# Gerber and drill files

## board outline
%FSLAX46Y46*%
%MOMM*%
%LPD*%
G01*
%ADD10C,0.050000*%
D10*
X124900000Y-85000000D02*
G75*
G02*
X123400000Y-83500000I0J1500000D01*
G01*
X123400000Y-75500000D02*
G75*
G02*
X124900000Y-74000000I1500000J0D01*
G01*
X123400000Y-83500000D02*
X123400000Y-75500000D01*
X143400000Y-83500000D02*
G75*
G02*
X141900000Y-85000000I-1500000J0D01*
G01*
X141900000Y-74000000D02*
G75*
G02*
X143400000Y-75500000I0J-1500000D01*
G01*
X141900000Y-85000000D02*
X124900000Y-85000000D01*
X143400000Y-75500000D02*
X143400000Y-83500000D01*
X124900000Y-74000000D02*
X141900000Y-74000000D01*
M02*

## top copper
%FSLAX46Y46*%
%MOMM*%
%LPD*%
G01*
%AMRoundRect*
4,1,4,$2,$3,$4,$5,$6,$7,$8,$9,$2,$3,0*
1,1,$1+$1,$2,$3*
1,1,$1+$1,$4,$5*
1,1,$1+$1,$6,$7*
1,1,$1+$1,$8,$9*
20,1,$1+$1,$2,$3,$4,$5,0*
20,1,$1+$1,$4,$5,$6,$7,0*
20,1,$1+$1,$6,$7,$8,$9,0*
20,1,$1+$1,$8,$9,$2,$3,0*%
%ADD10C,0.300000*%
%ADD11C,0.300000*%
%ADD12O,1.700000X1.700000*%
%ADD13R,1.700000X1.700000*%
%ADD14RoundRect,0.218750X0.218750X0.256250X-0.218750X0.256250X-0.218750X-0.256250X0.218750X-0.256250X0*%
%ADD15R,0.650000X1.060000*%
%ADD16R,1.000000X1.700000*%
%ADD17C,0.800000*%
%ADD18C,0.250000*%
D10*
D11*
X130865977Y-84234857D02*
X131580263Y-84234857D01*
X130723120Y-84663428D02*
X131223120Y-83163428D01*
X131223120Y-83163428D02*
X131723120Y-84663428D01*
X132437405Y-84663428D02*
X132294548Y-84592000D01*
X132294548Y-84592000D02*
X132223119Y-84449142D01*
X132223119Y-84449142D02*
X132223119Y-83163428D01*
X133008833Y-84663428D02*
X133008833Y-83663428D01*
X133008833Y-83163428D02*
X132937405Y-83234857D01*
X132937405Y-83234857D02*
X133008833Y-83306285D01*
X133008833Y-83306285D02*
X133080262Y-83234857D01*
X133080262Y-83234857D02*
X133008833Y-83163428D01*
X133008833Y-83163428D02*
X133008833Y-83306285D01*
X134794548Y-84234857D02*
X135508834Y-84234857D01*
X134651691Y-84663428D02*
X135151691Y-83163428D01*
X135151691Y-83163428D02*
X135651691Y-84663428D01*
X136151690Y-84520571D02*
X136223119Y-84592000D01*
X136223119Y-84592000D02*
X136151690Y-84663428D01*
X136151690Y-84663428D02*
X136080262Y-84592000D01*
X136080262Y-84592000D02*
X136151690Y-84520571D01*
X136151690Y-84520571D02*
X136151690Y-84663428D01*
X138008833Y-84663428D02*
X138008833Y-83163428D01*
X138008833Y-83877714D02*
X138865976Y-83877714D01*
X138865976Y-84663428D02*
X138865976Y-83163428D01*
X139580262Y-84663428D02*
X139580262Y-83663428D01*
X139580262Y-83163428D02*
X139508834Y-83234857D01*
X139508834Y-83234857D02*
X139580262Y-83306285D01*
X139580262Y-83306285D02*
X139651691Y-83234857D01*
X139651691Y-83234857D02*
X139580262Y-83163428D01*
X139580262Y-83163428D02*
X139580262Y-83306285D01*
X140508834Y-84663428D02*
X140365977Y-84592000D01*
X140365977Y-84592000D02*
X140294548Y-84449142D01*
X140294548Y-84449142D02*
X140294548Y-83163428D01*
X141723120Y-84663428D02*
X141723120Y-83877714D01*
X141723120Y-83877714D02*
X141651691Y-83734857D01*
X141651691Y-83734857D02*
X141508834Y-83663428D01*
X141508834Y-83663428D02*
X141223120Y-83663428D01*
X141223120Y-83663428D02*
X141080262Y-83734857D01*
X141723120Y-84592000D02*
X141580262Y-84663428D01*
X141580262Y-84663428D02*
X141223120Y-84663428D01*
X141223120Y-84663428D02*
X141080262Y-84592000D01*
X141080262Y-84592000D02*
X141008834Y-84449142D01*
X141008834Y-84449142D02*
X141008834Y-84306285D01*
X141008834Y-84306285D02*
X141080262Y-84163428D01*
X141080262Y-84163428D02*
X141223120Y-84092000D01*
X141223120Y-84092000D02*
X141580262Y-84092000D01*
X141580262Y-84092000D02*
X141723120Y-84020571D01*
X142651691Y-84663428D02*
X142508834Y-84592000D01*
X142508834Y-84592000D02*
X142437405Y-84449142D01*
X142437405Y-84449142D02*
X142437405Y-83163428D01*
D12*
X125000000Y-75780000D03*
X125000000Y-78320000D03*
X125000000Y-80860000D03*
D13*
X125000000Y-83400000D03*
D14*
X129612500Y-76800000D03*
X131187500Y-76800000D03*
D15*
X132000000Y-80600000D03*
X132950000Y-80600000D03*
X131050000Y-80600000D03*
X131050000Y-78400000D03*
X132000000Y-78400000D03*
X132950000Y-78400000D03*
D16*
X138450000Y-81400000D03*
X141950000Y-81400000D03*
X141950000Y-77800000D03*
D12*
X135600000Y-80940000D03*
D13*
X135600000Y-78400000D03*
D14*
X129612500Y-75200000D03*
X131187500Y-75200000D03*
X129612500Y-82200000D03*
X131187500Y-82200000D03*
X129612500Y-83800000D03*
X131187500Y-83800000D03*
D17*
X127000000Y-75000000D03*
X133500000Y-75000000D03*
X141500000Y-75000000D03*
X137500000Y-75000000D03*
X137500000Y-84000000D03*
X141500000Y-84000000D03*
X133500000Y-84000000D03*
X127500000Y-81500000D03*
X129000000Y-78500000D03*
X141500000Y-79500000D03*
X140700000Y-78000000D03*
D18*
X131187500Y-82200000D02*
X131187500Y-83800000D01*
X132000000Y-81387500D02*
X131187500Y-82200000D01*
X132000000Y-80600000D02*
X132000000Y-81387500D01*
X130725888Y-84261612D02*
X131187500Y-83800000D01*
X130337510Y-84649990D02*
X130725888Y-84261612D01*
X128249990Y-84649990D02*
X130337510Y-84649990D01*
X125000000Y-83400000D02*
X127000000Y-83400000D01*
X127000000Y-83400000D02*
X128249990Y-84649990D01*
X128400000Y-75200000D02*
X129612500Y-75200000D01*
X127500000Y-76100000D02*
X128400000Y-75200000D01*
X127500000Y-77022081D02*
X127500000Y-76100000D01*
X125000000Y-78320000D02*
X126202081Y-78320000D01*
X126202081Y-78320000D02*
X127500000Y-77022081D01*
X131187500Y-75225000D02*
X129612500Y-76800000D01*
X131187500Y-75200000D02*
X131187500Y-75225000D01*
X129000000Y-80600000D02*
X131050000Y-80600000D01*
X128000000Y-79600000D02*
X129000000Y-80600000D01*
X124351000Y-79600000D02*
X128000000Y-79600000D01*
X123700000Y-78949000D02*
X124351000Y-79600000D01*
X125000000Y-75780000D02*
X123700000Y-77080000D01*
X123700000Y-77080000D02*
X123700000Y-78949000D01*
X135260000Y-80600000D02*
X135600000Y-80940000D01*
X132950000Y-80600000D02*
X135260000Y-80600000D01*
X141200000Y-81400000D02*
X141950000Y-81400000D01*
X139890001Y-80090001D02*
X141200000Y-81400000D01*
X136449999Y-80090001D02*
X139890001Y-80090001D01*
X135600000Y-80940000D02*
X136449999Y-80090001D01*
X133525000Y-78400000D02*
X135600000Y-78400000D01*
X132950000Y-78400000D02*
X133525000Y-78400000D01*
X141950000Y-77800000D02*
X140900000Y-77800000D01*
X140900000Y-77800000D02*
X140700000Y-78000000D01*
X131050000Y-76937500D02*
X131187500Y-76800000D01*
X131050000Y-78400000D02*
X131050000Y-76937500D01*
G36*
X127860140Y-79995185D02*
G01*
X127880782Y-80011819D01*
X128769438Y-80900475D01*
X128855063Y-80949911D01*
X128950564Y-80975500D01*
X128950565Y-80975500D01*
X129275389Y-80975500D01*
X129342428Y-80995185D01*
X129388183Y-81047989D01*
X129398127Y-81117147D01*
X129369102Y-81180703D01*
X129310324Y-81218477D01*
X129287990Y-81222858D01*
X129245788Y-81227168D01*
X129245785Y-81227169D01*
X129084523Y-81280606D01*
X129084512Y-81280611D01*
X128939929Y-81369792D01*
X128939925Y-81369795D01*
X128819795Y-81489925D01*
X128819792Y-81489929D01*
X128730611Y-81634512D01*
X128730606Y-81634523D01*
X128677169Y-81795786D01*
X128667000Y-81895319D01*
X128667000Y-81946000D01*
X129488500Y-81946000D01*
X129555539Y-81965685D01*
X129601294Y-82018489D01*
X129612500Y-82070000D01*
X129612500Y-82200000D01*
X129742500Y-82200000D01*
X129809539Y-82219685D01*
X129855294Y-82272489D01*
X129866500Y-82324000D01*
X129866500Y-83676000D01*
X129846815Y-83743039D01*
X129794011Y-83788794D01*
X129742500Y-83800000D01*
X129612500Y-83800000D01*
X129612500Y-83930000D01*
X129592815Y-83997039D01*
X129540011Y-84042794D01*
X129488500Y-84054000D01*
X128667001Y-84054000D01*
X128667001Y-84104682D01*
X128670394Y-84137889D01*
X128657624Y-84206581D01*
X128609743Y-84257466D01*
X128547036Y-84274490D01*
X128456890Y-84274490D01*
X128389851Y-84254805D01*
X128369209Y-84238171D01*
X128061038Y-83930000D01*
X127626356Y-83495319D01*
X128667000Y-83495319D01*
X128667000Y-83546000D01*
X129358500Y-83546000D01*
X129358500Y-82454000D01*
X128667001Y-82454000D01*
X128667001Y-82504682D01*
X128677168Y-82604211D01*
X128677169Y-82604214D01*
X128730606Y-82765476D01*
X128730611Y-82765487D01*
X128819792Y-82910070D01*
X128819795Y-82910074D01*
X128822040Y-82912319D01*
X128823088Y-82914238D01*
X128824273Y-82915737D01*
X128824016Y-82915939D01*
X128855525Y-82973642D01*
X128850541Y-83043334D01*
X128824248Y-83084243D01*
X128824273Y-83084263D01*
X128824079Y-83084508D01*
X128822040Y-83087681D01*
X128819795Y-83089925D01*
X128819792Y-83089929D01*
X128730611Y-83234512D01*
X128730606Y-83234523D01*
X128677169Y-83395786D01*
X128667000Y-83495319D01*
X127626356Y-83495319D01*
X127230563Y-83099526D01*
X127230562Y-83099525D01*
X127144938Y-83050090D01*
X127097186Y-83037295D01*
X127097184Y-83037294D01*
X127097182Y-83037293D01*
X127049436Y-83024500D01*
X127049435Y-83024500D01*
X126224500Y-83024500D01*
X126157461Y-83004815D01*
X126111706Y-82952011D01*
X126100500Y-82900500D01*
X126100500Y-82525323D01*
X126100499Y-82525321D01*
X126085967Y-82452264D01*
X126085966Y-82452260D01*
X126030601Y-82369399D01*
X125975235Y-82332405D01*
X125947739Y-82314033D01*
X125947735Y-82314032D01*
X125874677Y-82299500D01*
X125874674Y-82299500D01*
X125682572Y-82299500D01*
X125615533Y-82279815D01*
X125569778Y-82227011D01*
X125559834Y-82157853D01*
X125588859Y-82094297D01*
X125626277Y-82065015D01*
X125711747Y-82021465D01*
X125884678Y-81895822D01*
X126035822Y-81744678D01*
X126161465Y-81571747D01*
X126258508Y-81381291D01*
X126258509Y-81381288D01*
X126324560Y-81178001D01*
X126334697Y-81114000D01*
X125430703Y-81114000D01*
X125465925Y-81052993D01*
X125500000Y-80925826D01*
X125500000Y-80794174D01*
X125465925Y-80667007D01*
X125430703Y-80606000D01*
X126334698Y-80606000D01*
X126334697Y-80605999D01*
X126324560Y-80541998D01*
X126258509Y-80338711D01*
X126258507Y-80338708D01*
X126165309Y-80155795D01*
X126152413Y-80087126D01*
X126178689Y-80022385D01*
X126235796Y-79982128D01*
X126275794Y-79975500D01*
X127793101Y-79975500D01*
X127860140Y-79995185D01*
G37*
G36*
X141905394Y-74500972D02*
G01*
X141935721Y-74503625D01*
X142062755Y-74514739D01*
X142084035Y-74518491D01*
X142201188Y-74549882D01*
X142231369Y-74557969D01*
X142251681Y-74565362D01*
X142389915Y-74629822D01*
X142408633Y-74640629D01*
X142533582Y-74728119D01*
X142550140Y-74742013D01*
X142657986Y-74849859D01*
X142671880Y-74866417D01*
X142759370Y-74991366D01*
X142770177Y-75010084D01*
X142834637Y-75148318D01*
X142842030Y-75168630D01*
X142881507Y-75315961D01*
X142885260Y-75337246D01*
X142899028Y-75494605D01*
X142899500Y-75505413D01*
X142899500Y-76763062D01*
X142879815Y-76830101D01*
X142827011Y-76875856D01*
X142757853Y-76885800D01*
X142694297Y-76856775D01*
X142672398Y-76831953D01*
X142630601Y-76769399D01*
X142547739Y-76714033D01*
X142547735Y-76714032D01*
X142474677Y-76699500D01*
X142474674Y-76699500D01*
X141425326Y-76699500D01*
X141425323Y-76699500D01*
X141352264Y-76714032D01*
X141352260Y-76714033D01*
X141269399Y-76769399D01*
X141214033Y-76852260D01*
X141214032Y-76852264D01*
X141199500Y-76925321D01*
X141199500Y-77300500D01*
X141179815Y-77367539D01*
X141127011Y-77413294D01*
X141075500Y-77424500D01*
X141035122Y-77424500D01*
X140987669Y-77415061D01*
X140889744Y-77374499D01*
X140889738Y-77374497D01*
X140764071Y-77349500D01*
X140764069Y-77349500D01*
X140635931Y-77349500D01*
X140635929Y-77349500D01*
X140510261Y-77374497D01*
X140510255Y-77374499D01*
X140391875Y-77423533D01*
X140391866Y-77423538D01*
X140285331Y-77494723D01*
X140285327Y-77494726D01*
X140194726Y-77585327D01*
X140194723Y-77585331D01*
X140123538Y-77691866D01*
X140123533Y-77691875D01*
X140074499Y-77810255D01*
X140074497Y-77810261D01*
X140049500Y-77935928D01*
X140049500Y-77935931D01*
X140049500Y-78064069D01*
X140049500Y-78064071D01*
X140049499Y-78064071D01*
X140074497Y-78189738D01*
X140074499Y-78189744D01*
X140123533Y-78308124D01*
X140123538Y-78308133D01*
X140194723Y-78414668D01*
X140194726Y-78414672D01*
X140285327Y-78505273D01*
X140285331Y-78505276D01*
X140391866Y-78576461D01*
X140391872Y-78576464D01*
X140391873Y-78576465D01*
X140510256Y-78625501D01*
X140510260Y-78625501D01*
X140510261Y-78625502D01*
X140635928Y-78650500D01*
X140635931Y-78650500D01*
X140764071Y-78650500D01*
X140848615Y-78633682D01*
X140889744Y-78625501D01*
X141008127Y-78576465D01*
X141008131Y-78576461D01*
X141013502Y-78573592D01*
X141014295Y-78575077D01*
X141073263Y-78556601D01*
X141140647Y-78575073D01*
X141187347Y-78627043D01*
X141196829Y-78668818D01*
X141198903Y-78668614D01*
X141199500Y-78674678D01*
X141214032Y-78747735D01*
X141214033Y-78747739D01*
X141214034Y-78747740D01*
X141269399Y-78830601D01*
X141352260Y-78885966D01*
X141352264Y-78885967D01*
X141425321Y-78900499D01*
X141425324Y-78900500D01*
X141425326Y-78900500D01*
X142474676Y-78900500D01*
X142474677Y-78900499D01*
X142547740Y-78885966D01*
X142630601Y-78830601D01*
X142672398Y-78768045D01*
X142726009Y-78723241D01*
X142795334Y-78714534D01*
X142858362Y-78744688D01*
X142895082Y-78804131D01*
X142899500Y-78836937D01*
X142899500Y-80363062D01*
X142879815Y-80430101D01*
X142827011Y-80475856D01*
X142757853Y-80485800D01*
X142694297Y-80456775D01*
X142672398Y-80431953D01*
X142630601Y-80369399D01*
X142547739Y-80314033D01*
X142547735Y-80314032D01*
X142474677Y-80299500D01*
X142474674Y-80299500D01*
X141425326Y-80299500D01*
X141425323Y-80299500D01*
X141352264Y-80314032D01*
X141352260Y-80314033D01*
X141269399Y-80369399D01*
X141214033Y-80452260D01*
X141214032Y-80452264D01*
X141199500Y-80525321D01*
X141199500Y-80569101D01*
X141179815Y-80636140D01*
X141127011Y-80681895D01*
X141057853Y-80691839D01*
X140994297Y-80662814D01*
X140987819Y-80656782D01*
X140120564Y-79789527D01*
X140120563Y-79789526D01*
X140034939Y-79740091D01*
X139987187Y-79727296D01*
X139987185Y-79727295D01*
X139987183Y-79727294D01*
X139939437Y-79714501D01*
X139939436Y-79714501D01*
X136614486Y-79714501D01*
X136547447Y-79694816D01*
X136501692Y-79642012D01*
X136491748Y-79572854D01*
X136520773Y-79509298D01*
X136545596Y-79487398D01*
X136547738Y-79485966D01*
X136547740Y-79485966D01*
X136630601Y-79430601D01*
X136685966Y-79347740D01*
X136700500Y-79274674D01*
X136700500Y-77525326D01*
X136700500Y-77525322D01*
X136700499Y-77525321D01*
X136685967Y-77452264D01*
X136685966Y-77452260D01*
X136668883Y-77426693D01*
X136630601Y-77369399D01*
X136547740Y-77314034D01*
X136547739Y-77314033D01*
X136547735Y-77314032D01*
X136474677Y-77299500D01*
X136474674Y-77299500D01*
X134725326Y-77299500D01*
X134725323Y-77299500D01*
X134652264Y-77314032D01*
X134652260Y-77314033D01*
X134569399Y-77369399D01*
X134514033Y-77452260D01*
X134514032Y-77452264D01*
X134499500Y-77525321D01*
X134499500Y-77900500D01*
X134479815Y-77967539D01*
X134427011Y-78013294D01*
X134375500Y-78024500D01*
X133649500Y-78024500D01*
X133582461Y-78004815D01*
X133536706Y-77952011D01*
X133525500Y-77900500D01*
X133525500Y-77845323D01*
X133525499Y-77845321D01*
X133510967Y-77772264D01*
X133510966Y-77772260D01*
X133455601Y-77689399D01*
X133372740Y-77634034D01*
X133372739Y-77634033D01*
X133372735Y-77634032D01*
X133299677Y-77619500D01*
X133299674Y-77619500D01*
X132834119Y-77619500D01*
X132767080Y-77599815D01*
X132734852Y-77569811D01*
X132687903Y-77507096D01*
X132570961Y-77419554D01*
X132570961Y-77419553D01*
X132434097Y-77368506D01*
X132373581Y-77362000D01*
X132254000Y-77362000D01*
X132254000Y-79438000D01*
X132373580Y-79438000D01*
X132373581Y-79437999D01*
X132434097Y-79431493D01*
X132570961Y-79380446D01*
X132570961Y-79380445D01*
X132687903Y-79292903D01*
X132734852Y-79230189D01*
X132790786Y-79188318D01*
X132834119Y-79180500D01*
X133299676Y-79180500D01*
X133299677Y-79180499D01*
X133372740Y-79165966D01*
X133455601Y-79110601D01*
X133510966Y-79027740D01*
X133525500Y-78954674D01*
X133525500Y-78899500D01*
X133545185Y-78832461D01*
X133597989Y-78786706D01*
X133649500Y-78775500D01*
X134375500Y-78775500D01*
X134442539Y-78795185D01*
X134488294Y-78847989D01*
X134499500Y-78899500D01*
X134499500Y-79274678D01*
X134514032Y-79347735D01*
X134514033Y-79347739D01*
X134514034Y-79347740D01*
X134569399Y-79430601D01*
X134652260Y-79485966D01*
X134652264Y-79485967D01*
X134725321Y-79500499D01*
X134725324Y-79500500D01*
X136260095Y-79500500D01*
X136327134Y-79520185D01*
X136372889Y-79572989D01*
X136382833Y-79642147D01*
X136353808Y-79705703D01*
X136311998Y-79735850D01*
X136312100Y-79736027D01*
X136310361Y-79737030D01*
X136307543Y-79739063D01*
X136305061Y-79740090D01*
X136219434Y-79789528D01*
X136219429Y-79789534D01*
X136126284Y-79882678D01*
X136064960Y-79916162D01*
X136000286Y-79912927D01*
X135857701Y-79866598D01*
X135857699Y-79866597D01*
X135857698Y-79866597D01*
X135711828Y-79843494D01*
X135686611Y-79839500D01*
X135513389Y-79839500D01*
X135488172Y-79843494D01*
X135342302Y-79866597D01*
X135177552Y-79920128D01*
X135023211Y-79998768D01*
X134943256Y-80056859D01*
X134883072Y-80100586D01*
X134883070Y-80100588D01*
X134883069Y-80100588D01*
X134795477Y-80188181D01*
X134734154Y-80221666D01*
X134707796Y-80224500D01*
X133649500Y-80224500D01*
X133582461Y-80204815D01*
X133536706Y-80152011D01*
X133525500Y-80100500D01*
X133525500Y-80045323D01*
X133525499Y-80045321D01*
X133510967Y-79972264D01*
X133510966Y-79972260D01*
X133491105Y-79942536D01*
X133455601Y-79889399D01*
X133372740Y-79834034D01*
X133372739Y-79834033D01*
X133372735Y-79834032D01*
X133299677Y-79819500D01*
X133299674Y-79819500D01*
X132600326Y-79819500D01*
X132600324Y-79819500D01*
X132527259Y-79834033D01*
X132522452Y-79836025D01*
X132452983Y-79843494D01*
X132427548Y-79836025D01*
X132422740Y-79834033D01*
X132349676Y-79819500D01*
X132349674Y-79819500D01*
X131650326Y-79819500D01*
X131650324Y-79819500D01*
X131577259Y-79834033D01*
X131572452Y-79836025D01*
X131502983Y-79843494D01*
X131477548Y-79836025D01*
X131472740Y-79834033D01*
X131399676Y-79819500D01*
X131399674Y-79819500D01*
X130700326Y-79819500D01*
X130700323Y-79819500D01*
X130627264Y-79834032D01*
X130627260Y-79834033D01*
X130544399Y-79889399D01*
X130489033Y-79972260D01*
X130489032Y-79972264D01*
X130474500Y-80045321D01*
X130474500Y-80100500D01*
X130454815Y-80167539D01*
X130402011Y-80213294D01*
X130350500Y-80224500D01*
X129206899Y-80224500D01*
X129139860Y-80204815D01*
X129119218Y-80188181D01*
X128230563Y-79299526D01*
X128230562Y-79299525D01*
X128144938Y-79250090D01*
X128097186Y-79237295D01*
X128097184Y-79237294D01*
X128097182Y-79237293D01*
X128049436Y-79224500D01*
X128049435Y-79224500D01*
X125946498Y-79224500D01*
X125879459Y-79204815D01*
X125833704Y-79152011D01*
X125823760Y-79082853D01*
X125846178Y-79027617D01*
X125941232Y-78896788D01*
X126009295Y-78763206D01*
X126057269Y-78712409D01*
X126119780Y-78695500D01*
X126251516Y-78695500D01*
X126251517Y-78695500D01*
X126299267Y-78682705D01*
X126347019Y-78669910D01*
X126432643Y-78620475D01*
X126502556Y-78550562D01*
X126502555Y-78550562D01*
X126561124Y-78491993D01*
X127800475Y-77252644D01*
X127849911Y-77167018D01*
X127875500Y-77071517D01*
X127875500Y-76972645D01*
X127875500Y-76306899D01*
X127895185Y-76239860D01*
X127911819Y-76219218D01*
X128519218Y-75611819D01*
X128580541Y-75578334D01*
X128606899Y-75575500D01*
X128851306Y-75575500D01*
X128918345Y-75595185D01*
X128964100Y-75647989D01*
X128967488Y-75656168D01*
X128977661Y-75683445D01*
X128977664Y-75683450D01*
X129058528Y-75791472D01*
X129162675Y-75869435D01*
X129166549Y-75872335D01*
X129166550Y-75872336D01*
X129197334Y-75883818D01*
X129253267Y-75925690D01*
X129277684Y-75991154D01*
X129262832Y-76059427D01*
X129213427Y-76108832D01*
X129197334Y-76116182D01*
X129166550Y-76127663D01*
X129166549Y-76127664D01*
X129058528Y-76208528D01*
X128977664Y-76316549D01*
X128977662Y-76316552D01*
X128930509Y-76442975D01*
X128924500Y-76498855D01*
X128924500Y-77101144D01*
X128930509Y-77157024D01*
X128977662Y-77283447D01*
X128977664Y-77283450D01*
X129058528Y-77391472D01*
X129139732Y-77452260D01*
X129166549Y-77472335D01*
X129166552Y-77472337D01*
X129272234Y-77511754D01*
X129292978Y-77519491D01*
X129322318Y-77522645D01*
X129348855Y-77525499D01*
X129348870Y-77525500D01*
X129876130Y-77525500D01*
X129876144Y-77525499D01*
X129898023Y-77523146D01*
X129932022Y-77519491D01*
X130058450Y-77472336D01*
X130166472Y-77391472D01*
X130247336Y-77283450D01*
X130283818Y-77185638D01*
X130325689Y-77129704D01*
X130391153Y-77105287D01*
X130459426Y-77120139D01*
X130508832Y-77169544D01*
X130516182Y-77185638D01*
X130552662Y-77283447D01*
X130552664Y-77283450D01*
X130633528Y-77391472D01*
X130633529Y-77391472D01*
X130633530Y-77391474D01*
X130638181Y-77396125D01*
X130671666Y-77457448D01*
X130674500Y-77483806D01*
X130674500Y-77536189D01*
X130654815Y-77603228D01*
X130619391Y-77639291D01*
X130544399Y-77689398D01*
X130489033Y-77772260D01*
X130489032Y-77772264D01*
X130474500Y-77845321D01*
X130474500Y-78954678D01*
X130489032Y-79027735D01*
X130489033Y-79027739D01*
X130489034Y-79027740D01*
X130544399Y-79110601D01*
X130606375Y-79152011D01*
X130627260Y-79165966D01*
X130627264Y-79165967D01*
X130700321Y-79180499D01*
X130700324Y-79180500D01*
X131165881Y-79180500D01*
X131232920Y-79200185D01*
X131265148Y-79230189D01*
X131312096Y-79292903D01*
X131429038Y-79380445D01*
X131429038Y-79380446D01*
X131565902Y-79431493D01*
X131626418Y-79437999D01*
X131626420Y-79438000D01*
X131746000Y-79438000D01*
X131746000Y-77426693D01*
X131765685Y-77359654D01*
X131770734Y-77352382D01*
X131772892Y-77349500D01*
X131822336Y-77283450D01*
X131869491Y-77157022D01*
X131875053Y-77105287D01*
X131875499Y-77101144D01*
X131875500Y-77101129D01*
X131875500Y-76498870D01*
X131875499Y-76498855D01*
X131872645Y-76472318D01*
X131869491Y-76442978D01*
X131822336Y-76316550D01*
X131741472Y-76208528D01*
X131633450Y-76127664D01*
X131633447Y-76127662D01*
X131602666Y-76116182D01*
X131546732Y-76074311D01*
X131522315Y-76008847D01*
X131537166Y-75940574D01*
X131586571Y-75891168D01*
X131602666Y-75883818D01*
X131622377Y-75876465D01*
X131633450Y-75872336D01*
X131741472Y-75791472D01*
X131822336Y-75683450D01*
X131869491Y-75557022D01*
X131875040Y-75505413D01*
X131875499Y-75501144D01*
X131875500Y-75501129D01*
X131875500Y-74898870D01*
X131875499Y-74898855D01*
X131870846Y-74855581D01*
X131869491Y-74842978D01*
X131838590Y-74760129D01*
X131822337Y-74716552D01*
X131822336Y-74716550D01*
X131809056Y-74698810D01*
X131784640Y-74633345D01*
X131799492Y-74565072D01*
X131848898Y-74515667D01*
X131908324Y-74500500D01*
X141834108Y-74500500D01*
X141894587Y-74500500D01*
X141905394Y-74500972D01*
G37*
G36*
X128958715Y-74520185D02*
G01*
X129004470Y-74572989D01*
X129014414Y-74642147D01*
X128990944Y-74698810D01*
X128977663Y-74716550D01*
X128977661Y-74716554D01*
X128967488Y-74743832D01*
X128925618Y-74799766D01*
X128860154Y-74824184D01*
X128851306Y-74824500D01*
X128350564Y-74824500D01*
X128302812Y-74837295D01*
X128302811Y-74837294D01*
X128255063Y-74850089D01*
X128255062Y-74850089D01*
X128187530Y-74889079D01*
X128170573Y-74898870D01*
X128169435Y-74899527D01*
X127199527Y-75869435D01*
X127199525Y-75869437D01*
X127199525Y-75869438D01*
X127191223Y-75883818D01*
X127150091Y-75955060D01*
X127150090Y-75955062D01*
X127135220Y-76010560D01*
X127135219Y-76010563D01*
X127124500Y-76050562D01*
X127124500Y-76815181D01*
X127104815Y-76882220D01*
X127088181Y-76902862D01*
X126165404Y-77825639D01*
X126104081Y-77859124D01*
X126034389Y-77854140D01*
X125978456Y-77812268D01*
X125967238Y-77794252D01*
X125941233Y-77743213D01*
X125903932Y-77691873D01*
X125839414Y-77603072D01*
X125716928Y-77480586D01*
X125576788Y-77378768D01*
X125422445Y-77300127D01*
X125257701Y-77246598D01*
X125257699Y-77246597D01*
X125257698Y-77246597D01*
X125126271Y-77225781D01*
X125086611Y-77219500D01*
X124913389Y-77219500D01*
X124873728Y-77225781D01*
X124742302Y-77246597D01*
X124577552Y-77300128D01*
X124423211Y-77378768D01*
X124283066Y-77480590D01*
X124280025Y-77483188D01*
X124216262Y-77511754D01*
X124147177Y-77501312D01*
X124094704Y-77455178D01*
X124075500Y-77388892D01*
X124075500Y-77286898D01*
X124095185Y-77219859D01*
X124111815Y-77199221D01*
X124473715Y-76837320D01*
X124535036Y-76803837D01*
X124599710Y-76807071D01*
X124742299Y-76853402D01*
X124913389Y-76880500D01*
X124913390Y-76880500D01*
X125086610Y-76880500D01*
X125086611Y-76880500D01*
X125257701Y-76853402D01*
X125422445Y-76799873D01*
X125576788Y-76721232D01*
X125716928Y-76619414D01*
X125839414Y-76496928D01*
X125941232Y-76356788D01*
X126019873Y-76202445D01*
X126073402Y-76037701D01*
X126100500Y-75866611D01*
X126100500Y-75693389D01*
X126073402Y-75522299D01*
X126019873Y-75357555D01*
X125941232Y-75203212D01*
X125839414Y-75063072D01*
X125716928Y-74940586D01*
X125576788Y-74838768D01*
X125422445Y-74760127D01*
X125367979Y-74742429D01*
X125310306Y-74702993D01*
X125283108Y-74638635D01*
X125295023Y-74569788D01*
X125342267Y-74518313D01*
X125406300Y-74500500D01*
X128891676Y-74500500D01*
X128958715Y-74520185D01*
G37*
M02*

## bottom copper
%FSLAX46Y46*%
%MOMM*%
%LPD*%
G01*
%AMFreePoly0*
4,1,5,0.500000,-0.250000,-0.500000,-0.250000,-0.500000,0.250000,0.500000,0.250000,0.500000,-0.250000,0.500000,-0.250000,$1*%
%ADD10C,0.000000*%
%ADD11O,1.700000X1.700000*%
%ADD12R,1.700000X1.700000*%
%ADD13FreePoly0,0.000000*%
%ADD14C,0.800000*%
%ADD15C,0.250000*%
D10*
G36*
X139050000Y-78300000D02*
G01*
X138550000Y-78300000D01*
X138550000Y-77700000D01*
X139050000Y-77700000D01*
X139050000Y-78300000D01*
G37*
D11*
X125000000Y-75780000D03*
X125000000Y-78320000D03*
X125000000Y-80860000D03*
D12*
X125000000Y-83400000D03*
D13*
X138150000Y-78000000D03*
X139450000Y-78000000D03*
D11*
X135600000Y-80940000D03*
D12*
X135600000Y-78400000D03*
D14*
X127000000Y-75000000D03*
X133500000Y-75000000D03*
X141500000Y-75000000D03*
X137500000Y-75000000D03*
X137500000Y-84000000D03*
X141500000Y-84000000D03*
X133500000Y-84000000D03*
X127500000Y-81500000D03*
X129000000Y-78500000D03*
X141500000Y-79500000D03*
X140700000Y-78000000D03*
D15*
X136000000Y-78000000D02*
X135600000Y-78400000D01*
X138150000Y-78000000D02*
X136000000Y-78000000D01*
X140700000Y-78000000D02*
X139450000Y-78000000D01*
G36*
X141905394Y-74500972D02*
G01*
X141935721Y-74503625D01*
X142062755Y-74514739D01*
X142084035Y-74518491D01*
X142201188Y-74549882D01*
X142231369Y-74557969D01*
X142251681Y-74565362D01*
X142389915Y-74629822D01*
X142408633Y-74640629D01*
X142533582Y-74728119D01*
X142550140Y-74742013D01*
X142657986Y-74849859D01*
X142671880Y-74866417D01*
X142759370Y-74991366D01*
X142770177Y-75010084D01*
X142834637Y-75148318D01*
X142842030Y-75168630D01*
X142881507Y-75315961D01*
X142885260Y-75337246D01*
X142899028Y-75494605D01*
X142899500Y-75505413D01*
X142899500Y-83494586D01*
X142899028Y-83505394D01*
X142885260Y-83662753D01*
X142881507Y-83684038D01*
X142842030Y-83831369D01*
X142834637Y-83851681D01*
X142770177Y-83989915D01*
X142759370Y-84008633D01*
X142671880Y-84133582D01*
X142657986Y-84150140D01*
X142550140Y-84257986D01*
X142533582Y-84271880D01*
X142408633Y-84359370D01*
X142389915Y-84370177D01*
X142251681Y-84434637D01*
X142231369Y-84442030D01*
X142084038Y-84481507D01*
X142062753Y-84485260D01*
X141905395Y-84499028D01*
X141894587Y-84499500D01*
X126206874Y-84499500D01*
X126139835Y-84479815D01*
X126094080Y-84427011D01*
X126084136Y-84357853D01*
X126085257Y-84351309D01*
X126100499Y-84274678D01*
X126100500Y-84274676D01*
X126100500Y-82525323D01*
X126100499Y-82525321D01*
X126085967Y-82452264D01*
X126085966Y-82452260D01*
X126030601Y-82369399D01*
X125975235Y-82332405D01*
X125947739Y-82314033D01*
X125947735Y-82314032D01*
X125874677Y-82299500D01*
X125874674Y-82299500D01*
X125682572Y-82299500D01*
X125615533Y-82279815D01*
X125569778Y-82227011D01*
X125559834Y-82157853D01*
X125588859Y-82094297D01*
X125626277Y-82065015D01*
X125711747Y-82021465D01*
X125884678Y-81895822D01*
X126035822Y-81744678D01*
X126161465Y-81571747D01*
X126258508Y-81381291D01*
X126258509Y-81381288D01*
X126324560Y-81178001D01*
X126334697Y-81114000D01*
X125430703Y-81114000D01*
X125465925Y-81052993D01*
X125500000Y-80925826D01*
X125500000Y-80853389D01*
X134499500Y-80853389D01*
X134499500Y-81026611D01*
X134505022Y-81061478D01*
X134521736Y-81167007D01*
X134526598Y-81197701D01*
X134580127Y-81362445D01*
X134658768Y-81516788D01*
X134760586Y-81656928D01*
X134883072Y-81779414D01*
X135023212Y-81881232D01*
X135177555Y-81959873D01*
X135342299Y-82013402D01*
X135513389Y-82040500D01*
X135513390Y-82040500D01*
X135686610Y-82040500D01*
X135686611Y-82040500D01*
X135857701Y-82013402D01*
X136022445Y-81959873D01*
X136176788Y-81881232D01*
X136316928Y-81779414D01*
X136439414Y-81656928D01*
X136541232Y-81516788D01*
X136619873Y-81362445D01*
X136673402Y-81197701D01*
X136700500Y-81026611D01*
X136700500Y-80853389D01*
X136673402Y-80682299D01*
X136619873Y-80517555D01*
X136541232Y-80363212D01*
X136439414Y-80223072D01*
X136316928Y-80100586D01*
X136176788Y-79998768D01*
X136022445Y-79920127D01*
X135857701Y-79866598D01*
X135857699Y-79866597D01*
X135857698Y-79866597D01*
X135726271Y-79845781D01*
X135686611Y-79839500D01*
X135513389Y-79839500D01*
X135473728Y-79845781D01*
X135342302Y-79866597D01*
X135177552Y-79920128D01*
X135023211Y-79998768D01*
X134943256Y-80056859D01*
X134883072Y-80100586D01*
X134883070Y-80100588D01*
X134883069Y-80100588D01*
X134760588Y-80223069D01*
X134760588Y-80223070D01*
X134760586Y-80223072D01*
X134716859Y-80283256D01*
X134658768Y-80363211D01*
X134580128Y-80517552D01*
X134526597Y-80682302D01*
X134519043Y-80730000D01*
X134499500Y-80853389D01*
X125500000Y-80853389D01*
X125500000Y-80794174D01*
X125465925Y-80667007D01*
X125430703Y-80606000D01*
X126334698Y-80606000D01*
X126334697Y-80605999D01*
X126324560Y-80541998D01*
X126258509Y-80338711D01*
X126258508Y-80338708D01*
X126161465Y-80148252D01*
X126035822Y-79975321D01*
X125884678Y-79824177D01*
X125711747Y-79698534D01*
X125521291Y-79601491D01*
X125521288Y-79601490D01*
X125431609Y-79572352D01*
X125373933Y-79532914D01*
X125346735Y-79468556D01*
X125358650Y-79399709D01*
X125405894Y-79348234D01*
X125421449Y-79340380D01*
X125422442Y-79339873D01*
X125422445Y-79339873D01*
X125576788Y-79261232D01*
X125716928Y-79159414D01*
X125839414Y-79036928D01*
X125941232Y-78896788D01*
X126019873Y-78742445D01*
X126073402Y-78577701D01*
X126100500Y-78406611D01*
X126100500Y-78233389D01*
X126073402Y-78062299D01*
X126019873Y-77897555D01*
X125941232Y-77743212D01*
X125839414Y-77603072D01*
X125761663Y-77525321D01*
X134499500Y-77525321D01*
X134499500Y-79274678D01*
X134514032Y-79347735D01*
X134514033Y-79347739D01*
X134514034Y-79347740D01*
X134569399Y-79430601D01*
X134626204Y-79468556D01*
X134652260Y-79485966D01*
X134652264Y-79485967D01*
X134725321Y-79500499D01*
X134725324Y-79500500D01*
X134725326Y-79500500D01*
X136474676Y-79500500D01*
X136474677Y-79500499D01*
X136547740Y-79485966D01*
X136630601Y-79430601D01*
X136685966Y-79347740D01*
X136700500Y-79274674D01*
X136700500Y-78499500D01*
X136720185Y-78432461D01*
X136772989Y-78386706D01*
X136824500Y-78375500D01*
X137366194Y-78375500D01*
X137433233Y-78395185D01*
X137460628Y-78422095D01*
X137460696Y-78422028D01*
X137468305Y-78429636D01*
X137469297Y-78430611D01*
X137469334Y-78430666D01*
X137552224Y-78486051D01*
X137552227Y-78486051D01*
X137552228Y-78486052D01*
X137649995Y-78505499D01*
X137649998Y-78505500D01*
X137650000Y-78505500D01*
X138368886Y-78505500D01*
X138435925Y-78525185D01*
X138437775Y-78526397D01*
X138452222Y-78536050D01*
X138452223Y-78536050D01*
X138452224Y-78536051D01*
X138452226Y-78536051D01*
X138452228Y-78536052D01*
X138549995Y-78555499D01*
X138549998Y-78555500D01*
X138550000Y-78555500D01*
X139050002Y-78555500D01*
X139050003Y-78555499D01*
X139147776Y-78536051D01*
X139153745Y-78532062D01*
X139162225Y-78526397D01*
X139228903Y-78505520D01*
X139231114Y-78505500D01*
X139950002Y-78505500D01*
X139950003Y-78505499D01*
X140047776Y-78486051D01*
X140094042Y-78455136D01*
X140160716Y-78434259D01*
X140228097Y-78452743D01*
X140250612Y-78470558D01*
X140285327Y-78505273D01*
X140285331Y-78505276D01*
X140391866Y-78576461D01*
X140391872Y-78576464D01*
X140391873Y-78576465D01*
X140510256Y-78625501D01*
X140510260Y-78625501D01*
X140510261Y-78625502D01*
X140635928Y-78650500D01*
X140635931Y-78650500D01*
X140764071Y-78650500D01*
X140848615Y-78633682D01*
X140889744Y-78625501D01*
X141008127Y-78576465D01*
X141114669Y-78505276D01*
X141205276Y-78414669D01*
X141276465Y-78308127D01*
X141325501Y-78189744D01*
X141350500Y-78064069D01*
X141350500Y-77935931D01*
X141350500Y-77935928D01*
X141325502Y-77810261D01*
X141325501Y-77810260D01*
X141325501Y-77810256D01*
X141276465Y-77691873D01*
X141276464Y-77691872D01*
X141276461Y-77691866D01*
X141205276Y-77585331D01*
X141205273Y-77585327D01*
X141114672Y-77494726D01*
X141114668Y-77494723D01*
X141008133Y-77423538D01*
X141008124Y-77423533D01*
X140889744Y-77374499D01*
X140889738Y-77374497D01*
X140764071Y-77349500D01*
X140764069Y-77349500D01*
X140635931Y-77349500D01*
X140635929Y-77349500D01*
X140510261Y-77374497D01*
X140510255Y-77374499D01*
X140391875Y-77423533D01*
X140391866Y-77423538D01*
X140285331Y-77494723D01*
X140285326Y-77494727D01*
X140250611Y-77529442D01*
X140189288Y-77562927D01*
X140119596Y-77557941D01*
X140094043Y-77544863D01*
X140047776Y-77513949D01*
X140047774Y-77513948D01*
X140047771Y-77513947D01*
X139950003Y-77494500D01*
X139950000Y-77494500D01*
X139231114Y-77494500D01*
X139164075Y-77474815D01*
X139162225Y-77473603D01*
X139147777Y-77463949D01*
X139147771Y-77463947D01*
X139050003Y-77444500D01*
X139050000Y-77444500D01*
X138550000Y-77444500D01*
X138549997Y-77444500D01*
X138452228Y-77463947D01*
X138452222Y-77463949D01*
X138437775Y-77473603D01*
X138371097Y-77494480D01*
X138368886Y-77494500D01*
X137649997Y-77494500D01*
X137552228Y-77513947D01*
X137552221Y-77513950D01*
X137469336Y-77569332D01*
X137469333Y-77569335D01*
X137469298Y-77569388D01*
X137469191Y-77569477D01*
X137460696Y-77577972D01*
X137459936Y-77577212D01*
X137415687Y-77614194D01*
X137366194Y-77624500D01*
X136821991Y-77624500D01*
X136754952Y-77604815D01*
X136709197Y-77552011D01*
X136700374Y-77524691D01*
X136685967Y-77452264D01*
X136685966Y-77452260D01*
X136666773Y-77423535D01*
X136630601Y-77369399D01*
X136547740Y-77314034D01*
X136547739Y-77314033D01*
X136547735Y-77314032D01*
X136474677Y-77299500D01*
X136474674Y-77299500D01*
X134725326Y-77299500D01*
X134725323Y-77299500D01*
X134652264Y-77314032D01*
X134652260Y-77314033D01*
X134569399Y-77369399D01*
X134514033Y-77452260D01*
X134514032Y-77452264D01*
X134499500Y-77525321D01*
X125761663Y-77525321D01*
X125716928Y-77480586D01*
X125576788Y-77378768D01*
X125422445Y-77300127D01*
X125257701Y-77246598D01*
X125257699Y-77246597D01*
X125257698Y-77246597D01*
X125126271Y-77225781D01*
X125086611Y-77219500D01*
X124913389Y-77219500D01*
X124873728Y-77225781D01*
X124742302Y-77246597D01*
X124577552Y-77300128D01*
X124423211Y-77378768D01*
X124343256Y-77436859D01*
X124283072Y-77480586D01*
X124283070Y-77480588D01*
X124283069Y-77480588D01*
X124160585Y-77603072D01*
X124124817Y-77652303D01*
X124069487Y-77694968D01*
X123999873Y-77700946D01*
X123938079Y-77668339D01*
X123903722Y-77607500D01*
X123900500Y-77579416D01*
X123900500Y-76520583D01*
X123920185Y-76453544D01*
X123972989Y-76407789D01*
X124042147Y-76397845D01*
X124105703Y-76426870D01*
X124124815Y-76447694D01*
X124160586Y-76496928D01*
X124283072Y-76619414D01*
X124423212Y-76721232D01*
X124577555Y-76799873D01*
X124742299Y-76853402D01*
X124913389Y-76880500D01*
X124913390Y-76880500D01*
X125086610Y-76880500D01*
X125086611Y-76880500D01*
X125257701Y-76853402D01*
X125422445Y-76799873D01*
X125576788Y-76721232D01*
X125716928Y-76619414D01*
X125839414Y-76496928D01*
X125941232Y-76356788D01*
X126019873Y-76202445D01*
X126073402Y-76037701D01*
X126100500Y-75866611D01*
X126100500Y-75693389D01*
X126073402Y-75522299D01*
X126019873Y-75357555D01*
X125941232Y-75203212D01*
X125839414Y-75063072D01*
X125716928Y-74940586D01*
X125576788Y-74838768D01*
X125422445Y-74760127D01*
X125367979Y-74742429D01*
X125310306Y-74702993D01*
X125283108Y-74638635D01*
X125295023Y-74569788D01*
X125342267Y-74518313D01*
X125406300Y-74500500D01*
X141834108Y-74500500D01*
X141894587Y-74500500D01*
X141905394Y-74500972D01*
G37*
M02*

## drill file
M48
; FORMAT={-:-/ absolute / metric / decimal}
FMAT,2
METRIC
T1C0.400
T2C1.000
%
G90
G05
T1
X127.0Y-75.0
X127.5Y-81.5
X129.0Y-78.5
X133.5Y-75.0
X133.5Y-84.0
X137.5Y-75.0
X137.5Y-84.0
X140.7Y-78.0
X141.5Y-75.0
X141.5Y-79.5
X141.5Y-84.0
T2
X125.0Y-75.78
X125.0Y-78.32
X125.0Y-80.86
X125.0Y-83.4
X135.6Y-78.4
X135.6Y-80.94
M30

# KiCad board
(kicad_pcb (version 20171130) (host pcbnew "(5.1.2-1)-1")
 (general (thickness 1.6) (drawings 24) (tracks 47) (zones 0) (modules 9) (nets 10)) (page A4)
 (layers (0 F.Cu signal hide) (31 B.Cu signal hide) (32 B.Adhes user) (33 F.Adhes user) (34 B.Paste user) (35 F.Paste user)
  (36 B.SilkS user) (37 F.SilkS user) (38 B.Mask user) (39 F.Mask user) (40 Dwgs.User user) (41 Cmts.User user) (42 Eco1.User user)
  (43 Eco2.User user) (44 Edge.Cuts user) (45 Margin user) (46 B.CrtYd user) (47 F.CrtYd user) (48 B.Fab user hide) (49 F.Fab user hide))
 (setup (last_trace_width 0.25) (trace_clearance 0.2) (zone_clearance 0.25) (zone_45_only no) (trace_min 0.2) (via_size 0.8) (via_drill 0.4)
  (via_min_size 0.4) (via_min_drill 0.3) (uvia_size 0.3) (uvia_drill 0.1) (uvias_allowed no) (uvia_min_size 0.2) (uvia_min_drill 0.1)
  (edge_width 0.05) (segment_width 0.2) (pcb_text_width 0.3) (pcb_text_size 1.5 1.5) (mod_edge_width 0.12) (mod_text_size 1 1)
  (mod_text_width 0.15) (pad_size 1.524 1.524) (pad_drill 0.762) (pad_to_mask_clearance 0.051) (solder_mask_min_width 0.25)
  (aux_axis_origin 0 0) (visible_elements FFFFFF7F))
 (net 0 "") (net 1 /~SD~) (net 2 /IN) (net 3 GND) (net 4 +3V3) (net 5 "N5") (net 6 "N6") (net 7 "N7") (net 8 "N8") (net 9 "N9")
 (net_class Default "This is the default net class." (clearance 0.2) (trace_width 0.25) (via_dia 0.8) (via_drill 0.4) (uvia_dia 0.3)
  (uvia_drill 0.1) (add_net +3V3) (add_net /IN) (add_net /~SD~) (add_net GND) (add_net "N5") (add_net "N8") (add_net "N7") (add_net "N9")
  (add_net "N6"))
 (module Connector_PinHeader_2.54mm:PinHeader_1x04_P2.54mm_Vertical (layer F.Cu) (at 125 83.4 180)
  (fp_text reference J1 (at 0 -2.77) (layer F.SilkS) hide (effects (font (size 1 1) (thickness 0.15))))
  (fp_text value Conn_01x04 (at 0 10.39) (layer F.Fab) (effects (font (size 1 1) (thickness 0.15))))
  (pad 4 thru_hole oval (at 0 7.62 180) (size 1.7 1.7) (drill 1) (layers *.Cu *.Mask) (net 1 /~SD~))
  (pad 3 thru_hole oval (at 0 5.08 180) (size 1.7 1.7) (drill 1) (layers *.Cu *.Mask) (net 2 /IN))
  (pad 2 thru_hole oval (at 0 2.54 180) (size 1.7 1.7) (drill 1) (layers *.Cu *.Mask) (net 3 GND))
  (pad 1 thru_hole rect (at 0 0 180) (size 1.7 1.7) (drill 1) (layers *.Cu *.Mask) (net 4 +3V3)))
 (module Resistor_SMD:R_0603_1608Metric (layer F.Cu) (at 130.4 76.8 180)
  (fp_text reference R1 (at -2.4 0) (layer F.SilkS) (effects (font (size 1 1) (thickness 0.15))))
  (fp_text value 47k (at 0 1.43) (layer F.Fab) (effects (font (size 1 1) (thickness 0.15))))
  (pad 2 smd roundrect (at 0.7875 0 180) (size 0.875 0.95) (layers F.Cu F.Paste F.Mask) (roundrect_rratio 0.25) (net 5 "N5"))
  (pad 1 smd roundrect (at -0.7875 0 180) (size 0.875 0.95) (layers F.Cu F.Paste F.Mask) (roundrect_rratio 0.25) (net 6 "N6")))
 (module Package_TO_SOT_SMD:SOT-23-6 (layer F.Cu) (at 132 79.5 270)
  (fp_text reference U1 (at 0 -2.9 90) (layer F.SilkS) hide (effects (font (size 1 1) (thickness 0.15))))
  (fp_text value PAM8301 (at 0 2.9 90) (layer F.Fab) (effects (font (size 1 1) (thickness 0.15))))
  (pad 5 smd rect (at 1.1 0 270) (size 1.06 0.65) (layers F.Cu F.Paste F.Mask) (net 4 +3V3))
  (pad 6 smd rect (at 1.1 -0.95 270) (size 1.06 0.65) (layers F.Cu F.Paste F.Mask) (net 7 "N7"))
  (pad 4 smd rect (at 1.1 0.95 270) (size 1.06 0.65) (layers F.Cu F.Paste F.Mask) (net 1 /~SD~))
  (pad 3 smd rect (at -1.1 0.95 270) (size 1.06 0.65) (layers F.Cu F.Paste F.Mask) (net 6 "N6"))
  (pad 2 smd rect (at -1.1 0 270) (size 1.06 0.65) (layers F.Cu F.Paste F.Mask) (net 3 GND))
  (pad 1 smd rect (at -1.1 -0.95 270) (size 1.06 0.65) (layers F.Cu F.Paste F.Mask) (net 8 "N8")))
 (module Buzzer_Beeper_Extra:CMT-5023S (layer F.Cu) (at 140.2 79.6 90)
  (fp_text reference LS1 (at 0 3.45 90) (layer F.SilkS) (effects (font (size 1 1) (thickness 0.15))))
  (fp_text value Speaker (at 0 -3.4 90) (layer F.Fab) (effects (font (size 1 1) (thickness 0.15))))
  (pad "" smd rect (at -1.8 -1.75 90) (size 1.7 1) (layers F.Cu F.Paste F.Mask))
  (pad 1 smd rect (at -1.8 1.75 90) (size 1.7 1) (layers F.Cu F.Paste F.Mask) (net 7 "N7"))
  (pad 2 smd rect (at 1.8 1.75 90) (size 1.7 1) (layers F.Cu F.Paste F.Mask) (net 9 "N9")))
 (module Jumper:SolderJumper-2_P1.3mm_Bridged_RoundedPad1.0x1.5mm (layer B.Cu) (at 138.8 78)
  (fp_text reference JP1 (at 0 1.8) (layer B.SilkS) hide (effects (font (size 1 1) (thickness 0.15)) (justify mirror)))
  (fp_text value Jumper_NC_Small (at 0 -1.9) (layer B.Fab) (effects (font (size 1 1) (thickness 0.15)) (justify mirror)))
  (fp_poly (pts (xy 0.25 0.3) (xy -0.25 0.3) (xy -0.25 -0.3) (xy 0.25 -0.3)) (layer B.Cu) (width 0))
  (pad 1 smd custom (at -0.65 0) (size 1 0.5) (layers B.Cu B.Mask) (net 8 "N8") (zone_connect 2) (options (clearance outline) (anchor rect))
   (primitives))
  (pad 2 smd custom (at 0.65 0) (size 1 0.5) (layers B.Cu B.Mask) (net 9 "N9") (zone_connect 2) (options (clearance outline) (anchor rect))
   (primitives)))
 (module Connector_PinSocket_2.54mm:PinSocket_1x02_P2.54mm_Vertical (layer F.Cu) (at 135.6 78.4)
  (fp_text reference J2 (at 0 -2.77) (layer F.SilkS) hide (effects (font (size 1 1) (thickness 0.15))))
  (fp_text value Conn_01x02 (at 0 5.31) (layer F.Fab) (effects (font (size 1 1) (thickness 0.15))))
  (pad 2 thru_hole oval (at 0 2.54) (size 1.7 1.7) (drill 1) (layers *.Cu *.Mask) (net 7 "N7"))
  (pad 1 thru_hole rect (at 0 0) (size 1.7 1.7) (drill 1) (layers *.Cu *.Mask) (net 8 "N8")))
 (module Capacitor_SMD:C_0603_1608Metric (layer F.Cu) (at 130.4 75.2 180)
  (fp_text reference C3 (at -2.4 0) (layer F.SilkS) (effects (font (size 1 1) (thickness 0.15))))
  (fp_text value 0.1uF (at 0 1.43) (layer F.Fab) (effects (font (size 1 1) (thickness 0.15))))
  (pad 2 smd roundrect (at 0.7875 0 180) (size 0.875 0.95) (layers F.Cu F.Paste F.Mask) (roundrect_rratio 0.25) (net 2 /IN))
  (pad 1 smd roundrect (at -0.7875 0 180) (size 0.875 0.95) (layers F.Cu F.Paste F.Mask) (roundrect_rratio 0.25) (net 5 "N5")))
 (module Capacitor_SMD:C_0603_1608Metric (layer F.Cu) (at 130.4 82.2 180)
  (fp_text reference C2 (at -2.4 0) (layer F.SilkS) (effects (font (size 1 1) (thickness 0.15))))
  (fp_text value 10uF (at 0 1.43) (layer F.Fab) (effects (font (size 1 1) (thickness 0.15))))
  (pad 2 smd roundrect (at 0.7875 0 180) (size 0.875 0.95) (layers F.Cu F.Paste F.Mask) (roundrect_rratio 0.25) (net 3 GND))
  (pad 1 smd roundrect (at -0.7875 0 180) (size 0.875 0.95) (layers F.Cu F.Paste F.Mask) (roundrect_rratio 0.25) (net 4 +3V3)))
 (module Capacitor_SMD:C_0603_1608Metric (layer F.Cu) (at 130.4 83.8 180)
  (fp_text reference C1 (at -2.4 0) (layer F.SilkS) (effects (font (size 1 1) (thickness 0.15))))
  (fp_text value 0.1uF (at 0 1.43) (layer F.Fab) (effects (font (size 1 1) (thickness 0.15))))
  (pad 2 smd roundrect (at 0.7875 0 180) (size 0.875 0.95) (layers F.Cu F.Paste F.Mask) (roundrect_rratio 0.25) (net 3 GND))
  (pad 1 smd roundrect (at -0.7875 0 180) (size 0.875 0.95) (layers F.Cu F.Paste F.Mask) (roundrect_rratio 0.25) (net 4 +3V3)))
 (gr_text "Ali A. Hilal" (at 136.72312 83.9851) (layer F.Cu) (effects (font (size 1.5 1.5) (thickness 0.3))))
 (gr_arc (start 124.9 83.5) (end 123.4 83.5) (angle -90) (layer Edge.Cuts) (width 0.05))
 (gr_arc (start 124.9 75.5) (end 124.9 74) (angle -90) (layer Edge.Cuts) (width 0.05))
 (gr_line (start 123.4 83.5) (end 123.4 75.5) (layer Edge.Cuts) (width 0.05))
 (gr_arc (start 141.9 83.5) (end 141.9 85) (angle -90) (layer Edge.Cuts) (width 0.05))
 (gr_arc (start 141.9 75.5) (end 143.4 75.5) (angle -90) (layer Edge.Cuts) (width 0.05))
 (gr_line (start 141.9 85) (end 124.9 85) (layer Edge.Cuts) (width 0.05))
 (gr_line (start 143.4 75.5) (end 143.4 83.5) (layer Edge.Cuts) (width 0.05))
 (gr_line (start 124.9 74) (end 141.9 74) (layer Edge.Cuts) (width 0.05))
 (via (at 127 75) (size 0.8) (drill 0.4) (layers F.Cu B.Cu) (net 3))
 (via (at 133.5 75) (size 0.8) (drill 0.4) (layers F.Cu B.Cu) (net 3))
 (via (at 141.5 75) (size 0.8) (drill 0.4) (layers F.Cu B.Cu) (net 3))
 (via (at 137.5 75) (size 0.8) (drill 0.4) (layers F.Cu B.Cu) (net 3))
 (via (at 137.5 84) (size 0.8) (drill 0.4) (layers F.Cu B.Cu) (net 3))
 (via (at 141.5 84) (size 0.8) (drill 0.4) (layers F.Cu B.Cu) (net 3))
 (via (at 133.5 84) (size 0.8) (drill 0.4) (layers F.Cu B.Cu) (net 3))
 (via (at 127.5 81.5) (size 0.8) (drill 0.4) (layers F.Cu B.Cu) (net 3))
 (via (at 129 78.5) (size 0.8) (drill 0.4) (layers F.Cu B.Cu) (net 3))
 (via (at 141.5 79.5) (size 0.8) (drill 0.4) (layers F.Cu B.Cu) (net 3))
 (segment (start 131.1875 82.2) (end 131.1875 83.8) (width 0.25) (layer F.Cu) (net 4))
 (segment (start 132 81.3875) (end 131.1875 82.2) (width 0.25) (layer F.Cu) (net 4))
 (segment (start 132 80.6) (end 132 81.3875) (width 0.25) (layer F.Cu) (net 4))
 (segment (start 130.725888 84.261612) (end 131.1875 83.8) (width 0.25) (layer F.Cu) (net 4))
 (segment (start 130.33751 84.64999) (end 130.725888 84.261612) (width 0.25) (layer F.Cu) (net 4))
 (segment (start 128.24999 84.64999) (end 130.33751 84.64999) (width 0.25) (layer F.Cu) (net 4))
 (segment (start 125 83.4) (end 127 83.4) (width 0.25) (layer F.Cu) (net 4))
 (segment (start 127 83.4) (end 128.24999 84.64999) (width 0.25) (layer F.Cu) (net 4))
 (segment (start 128.4 75.2) (end 129.6125 75.2) (width 0.25) (layer F.Cu) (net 2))
 (segment (start 127.5 76.1) (end 128.4 75.2) (width 0.25) (layer F.Cu) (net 2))
 (segment (start 127.5 77.022081) (end 127.5 76.1) (width 0.25) (layer F.Cu) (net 2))
 (segment (start 125 78.32) (end 126.202081 78.32) (width 0.25) (layer F.Cu) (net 2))
 (segment (start 126.202081 78.32) (end 127.5 77.022081) (width 0.25) (layer F.Cu) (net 2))
 (segment (start 131.1875 75.225) (end 129.6125 76.8) (width 0.25) (layer F.Cu) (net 5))
 (segment (start 131.1875 75.2) (end 131.1875 75.225) (width 0.25) (layer F.Cu) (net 5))
 (segment (start 129 80.6) (end 131.05 80.6) (width 0.25) (layer F.Cu) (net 1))
 (segment (start 128 79.6) (end 129 80.6) (width 0.25) (layer F.Cu) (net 1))
 (segment (start 124.351 79.6) (end 128 79.6) (width 0.25) (layer F.Cu) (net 1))
 (segment (start 123.7 78.949) (end 124.351 79.6) (width 0.25) (layer F.Cu) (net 1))
 (segment (start 125 75.78) (end 123.7 77.08) (width 0.25) (layer F.Cu) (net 1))
 (segment (start 123.7 77.08) (end 123.7 78.949) (width 0.25) (layer F.Cu) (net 1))
 (segment (start 135.26 80.6) (end 135.6 80.94) (width 0.25) (layer F.Cu) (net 7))
 (segment (start 132.95 80.6) (end 135.26 80.6) (width 0.25) (layer F.Cu) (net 7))
 (segment (start 141.2 81.4) (end 141.95 81.4) (width 0.25) (layer F.Cu) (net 7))
 (segment (start 139.890001 80.090001) (end 141.2 81.4) (width 0.25) (layer F.Cu) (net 7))
 (segment (start 136.449999 80.090001) (end 139.890001 80.090001) (width 0.25) (layer F.Cu) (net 7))
 (segment (start 135.6 80.94) (end 136.449999 80.090001) (width 0.25) (layer F.Cu) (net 7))
 (segment (start 133.525 78.4) (end 135.6 78.4) (width 0.25) (layer F.Cu) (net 8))
 (segment (start 132.95 78.4) (end 133.525 78.4) (width 0.25) (layer F.Cu) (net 8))
 (segment (start 136 78) (end 135.6 78.4) (width 0.25) (layer B.Cu) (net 8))
 (segment (start 138.15 78) (end 136 78) (width 0.25) (layer B.Cu) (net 8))
 (via (at 140.7 78) (size 0.8) (drill 0.4) (layers F.Cu B.Cu) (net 9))
 (segment (start 141.95 77.8) (end 140.9 77.8) (width 0.25) (layer F.Cu) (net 9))
 (segment (start 140.9 77.8) (end 140.7 78) (width 0.25) (layer F.Cu) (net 9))
 (segment (start 140.7 78) (end 139.45 78) (width 0.25) (layer B.Cu) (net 9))
 (segment (start 131.05 76.9375) (end 131.1875 76.8) (width 0.25) (layer F.Cu) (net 6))
 (segment (start 131.05 78.4) (end 131.05 76.9375) (width 0.25) (layer F.Cu) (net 6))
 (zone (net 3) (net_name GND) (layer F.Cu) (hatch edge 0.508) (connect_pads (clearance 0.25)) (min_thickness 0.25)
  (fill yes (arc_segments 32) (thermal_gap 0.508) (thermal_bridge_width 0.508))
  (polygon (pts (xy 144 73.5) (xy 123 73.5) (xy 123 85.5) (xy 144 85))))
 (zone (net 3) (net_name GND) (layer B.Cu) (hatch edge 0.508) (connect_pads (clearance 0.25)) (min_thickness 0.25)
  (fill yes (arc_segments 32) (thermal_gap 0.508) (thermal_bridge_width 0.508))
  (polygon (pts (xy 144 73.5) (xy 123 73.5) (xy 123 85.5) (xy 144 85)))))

